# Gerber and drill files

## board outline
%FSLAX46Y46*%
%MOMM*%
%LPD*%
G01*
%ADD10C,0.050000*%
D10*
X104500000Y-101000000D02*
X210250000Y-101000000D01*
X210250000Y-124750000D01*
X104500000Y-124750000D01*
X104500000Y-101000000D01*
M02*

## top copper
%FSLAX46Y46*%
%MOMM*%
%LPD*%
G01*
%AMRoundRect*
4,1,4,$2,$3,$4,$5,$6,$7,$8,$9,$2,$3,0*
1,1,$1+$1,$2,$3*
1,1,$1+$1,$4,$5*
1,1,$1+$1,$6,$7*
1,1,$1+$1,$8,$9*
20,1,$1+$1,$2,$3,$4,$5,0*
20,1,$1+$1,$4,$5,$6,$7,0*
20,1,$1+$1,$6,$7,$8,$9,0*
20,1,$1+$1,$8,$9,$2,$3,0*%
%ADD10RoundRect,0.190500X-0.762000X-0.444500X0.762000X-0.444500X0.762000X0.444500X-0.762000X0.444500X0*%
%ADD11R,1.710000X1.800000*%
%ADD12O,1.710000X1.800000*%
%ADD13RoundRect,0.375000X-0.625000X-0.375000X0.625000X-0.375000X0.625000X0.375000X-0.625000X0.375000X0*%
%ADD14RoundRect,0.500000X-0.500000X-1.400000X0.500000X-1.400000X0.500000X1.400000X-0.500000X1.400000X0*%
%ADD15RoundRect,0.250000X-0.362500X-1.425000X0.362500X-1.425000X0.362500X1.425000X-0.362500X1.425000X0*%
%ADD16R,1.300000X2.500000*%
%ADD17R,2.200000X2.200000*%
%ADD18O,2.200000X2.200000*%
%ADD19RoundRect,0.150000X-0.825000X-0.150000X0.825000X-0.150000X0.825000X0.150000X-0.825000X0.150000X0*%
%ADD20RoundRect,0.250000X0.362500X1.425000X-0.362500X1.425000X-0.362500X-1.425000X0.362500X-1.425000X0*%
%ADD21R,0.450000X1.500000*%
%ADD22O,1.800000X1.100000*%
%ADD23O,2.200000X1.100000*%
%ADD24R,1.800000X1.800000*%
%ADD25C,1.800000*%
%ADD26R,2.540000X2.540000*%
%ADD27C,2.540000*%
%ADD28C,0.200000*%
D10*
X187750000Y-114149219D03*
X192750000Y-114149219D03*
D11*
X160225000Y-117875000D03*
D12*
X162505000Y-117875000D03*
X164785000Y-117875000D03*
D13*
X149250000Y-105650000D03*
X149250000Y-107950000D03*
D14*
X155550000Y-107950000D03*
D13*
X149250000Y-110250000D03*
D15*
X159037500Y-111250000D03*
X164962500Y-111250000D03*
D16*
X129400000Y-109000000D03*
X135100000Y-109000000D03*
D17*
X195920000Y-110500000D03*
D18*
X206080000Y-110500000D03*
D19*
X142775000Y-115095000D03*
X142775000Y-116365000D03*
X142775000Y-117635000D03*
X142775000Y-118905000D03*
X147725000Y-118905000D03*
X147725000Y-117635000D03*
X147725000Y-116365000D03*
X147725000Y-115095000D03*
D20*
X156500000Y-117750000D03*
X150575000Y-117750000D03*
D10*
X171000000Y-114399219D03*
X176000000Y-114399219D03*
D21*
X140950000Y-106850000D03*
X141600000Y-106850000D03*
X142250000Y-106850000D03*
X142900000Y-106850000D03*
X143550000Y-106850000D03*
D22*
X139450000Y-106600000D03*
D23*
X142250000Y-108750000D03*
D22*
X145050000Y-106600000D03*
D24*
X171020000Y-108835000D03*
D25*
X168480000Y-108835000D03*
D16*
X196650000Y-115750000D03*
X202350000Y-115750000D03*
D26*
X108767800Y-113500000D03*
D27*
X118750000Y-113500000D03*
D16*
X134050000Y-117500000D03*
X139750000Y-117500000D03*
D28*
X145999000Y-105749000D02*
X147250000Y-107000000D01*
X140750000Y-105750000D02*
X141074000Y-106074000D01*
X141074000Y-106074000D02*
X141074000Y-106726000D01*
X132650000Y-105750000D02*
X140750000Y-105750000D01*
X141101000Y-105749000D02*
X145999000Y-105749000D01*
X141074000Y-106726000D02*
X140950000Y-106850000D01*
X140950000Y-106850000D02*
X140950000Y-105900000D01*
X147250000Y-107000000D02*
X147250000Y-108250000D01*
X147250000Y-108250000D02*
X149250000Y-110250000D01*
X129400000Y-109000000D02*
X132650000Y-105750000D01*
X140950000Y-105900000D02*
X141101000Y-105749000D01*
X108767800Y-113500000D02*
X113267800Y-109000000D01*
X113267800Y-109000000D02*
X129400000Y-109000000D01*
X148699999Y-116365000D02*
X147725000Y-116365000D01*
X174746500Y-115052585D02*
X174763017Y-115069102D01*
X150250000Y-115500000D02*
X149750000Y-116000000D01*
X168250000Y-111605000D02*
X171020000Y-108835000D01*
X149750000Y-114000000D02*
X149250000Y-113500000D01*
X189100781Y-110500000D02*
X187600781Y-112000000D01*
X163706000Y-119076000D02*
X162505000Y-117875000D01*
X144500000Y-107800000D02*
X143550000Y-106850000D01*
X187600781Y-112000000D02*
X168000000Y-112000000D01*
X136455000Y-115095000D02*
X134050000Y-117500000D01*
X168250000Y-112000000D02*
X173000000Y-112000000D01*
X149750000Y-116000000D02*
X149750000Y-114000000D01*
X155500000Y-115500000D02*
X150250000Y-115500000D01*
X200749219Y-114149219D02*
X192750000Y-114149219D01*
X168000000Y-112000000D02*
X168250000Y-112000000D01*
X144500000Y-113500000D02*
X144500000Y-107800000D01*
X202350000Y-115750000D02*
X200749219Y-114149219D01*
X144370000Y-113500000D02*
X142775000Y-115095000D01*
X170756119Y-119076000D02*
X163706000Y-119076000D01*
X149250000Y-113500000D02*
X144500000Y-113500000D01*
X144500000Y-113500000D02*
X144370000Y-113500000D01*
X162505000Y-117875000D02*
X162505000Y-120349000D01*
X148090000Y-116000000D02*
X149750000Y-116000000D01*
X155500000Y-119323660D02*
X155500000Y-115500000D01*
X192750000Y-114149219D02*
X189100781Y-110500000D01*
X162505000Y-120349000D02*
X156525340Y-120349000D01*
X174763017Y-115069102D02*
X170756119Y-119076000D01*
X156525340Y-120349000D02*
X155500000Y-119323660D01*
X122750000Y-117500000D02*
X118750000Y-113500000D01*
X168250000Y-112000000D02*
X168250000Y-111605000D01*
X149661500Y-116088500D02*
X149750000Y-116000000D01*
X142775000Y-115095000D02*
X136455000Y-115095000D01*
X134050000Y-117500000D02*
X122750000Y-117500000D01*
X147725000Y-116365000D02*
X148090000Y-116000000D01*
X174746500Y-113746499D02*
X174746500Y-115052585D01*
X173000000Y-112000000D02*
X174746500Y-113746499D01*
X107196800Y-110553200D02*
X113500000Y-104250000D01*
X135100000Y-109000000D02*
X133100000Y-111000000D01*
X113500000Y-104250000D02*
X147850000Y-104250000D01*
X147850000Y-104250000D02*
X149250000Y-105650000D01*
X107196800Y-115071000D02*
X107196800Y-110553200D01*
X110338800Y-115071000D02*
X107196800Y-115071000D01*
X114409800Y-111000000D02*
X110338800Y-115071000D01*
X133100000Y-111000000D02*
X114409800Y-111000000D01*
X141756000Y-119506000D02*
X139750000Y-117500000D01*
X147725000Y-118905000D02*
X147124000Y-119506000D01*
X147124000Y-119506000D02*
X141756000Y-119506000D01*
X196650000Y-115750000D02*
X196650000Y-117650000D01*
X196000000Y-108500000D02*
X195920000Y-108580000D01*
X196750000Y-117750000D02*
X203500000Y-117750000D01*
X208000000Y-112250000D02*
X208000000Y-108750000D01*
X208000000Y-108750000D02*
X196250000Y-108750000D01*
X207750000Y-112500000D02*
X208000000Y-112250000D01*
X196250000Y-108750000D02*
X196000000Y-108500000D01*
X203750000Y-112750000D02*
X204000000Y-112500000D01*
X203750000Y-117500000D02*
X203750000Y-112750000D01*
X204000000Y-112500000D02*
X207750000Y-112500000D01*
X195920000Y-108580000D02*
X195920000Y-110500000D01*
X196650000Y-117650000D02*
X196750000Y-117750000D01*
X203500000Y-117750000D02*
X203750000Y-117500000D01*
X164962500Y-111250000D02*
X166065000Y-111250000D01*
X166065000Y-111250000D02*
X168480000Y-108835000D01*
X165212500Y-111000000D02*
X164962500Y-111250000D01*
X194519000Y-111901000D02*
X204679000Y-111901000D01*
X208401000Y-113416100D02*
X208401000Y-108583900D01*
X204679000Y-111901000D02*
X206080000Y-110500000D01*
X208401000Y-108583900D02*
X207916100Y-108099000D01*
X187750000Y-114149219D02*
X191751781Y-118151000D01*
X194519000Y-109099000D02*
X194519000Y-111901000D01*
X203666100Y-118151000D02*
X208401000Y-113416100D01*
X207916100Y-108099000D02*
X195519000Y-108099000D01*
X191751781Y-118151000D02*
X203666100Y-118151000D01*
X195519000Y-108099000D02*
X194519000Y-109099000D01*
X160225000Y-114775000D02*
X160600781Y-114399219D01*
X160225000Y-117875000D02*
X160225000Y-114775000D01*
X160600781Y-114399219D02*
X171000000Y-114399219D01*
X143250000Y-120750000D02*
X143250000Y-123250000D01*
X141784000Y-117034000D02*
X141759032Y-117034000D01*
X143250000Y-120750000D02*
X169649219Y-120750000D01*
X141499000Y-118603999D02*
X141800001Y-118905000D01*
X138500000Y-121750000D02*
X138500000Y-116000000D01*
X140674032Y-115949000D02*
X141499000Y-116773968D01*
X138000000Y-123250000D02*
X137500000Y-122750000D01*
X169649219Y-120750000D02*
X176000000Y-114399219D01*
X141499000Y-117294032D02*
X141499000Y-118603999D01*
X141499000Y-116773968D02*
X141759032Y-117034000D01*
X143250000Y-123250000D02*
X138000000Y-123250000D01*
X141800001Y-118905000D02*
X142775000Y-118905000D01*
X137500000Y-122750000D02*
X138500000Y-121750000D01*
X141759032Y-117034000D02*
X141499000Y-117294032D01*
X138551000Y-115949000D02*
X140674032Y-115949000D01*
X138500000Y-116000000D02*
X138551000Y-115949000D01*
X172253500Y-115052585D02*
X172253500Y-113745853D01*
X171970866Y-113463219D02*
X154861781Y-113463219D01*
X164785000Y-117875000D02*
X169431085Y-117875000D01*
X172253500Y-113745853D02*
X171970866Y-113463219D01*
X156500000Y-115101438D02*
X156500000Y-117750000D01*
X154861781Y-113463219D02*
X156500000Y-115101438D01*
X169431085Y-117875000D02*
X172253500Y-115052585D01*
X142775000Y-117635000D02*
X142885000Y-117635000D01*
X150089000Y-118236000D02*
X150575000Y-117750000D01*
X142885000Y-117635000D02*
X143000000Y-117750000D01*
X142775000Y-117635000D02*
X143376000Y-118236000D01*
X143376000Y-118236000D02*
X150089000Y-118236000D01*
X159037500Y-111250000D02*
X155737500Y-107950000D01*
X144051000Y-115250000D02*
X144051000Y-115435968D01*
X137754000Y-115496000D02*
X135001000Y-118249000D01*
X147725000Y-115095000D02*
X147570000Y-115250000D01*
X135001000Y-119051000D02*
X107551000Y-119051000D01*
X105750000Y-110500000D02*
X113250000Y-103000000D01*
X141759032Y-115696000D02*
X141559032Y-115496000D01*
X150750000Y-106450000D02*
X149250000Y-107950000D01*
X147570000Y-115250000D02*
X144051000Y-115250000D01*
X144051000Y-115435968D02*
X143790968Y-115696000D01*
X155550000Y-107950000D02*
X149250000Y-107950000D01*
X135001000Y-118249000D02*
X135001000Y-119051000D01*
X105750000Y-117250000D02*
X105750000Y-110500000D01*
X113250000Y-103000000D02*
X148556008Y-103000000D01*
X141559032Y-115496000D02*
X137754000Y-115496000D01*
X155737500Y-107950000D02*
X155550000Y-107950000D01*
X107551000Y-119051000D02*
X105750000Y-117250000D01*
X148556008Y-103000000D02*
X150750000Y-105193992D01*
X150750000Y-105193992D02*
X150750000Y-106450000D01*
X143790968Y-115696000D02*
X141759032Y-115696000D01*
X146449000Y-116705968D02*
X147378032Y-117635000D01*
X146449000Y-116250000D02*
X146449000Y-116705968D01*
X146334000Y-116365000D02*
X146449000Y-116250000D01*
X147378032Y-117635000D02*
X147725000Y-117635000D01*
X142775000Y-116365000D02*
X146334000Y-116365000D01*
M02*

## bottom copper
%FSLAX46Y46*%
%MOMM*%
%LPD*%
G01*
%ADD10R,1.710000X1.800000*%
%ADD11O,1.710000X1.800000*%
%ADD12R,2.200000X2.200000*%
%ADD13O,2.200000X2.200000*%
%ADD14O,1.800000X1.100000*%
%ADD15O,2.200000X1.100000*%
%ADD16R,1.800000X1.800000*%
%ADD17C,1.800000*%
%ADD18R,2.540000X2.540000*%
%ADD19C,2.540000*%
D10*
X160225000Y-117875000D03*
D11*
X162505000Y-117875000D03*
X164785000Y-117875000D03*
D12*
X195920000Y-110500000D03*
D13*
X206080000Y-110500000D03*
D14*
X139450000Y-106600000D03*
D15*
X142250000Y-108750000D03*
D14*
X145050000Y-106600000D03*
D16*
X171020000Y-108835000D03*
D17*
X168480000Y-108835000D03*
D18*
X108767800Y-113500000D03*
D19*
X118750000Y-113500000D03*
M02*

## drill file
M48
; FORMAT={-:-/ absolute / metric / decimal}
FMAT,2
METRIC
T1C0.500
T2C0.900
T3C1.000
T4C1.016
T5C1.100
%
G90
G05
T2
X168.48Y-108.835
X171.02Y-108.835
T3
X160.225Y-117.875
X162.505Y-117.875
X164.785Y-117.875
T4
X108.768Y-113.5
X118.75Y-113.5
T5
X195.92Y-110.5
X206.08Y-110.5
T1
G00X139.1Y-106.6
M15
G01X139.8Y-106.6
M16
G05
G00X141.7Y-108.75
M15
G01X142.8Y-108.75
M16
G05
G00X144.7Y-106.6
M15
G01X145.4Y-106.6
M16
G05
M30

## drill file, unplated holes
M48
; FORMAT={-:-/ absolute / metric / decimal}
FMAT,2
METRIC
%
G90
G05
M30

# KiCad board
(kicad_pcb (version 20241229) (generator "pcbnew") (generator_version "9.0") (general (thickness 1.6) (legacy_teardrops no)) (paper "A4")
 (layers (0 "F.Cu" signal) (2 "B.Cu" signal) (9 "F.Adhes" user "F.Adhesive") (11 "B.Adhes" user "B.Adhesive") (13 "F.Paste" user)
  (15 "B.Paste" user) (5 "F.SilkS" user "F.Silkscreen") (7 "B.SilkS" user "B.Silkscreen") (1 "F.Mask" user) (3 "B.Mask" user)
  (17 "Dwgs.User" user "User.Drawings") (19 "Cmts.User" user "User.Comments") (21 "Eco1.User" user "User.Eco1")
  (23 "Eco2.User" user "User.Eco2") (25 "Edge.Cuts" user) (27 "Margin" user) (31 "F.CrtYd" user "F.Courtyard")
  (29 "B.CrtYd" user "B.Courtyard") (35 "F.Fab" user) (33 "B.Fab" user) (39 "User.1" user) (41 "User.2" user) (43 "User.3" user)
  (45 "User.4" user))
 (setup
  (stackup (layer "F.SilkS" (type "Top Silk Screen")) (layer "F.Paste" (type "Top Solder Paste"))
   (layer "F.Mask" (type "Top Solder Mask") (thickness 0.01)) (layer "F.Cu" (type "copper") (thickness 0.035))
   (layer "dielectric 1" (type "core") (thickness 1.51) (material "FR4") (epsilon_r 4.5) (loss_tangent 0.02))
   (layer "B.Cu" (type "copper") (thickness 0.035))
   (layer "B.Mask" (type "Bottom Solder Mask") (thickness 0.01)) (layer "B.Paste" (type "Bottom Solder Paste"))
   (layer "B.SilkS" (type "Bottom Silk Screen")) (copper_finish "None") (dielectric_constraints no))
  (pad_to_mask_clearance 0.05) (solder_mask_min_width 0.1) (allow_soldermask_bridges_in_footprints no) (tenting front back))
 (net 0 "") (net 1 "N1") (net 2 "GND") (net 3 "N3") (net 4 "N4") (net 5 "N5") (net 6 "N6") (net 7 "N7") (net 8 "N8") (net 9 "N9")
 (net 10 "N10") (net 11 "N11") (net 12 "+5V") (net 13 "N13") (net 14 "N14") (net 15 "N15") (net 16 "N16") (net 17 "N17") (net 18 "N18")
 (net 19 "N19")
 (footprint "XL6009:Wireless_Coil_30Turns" (layer "F.Cu") (at 190.25 109.149219)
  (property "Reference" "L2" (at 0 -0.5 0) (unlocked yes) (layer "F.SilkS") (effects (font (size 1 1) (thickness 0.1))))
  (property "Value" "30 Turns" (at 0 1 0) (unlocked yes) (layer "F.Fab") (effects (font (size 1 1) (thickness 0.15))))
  (pad "1" smd roundrect (at -2.5 5) (size 1.905 1.27) (layers "F.Cu" "F.Mask" "F.Paste") (roundrect_rratio 0.15) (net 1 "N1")
   (thermal_bridge_angle 45))
  (pad "2" smd roundrect (at 2.5 5) (size 1.905 1.27) (layers "F.Cu" "F.Mask" "F.Paste") (roundrect_rratio 0.15) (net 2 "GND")
   (thermal_bridge_angle 45)))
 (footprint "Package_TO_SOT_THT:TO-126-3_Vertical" (layer "F.Cu") (at 160.225 117.875)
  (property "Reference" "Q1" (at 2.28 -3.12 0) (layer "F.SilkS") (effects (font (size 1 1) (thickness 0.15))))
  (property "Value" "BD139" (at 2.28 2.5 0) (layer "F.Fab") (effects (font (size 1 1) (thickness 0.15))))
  (pad "1" thru_hole rect (at 0 0) (size 1.71 1.8) (drill 1) (layers "*.Cu" "*.Mask") (remove_unused_layers no) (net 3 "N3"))
  (pad "2" thru_hole oval (at 2.28 0) (size 1.71 1.8) (drill 1) (layers "*.Cu" "*.Mask") (remove_unused_layers no) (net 2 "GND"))
  (pad "3" thru_hole oval (at 4.56 0) (size 1.71 1.8) (drill 1) (layers "*.Cu" "*.Mask") (remove_unused_layers no) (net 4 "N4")))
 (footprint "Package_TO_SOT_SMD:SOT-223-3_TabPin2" (layer "F.Cu") (at 152.4 107.95)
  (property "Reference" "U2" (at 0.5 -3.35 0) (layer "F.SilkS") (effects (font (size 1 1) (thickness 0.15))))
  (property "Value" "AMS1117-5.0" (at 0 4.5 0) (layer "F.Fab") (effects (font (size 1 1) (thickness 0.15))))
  (pad "1" smd roundrect (at -3.15 -2.3) (size 2 1.5) (layers "F.Cu" "F.Mask" "F.Paste") (roundrect_rratio 0.25) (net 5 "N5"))
  (pad "2" smd roundrect (at -3.15 0) (size 2 1.5) (layers "F.Cu" "F.Mask" "F.Paste") (roundrect_rratio 0.25) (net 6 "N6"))
  (pad "2" smd roundrect (at 3.15 0) (size 2 3.8) (layers "F.Cu" "F.Mask" "F.Paste") (roundrect_rratio 0.25) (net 6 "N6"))
  (pad "3" smd roundrect (at -3.15 2.3) (size 2 1.5) (layers "F.Cu" "F.Mask" "F.Paste") (roundrect_rratio 0.25) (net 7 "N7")))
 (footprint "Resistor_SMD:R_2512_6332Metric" (layer "F.Cu") (at 162 111.25)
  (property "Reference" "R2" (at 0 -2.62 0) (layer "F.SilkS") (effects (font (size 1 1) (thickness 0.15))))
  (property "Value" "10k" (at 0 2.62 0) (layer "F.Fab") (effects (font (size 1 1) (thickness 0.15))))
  (pad "1" smd roundrect (at -2.9625 0) (size 1.225 3.35) (layers "F.Cu" "F.Mask" "F.Paste") (roundrect_rratio 0.204082) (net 6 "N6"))
  (pad "2" smd roundrect (at 2.9625 0) (size 1.225 3.35) (layers "F.Cu" "F.Mask" "F.Paste") (roundrect_rratio 0.204082) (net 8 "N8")))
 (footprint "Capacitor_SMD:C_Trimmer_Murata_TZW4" (layer "F.Cu") (at 132.25 109)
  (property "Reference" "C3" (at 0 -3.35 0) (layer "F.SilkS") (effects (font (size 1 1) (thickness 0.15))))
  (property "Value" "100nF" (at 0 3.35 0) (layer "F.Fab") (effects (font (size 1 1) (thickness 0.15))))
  (pad "1" smd rect (at -2.85 0) (size 1.3 2.5) (layers "F.Cu" "F.Mask" "F.Paste") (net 7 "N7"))
  (pad "2" smd rect (at 2.85 0) (size 1.3 2.5) (layers "F.Cu" "F.Mask" "F.Paste") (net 5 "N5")))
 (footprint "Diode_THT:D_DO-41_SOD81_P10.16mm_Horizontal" (layer "F.Cu") (at 195.92 110.5)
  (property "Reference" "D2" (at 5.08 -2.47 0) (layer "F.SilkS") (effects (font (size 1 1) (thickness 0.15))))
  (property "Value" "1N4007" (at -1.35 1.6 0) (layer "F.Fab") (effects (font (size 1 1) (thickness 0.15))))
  (pad "1" thru_hole rect (at 0 0) (size 2.2 2.2) (drill 1.1) (layers "*.Cu" "*.Mask") (remove_unused_layers no) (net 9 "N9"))
  (pad "2" thru_hole oval (at 10.16 0) (size 2.2 2.2) (drill 1.1) (layers "*.Cu" "*.Mask") (remove_unused_layers no) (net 1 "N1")))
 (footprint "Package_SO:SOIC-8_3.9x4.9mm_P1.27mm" (layer "F.Cu") (at 145.25 117)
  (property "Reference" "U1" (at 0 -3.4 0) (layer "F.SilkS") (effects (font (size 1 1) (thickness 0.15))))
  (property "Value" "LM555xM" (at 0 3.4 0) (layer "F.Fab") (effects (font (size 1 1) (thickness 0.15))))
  (pad "1" smd roundrect (at -2.475 -1.905) (size 1.95 0.6) (layers "F.Cu" "F.Mask" "F.Paste") (roundrect_rratio 0.25) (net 2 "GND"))
  (pad "2" smd roundrect (at -2.475 -0.635) (size 1.95 0.6) (layers "F.Cu" "F.Mask" "F.Paste") (roundrect_rratio 0.25) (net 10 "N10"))
  (pad "3" smd roundrect (at -2.475 0.635) (size 1.95 0.6) (layers "F.Cu" "F.Mask" "F.Paste") (roundrect_rratio 0.25) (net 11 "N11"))
  (pad "4" smd roundrect (at -2.475 1.905) (size 1.95 0.6) (layers "F.Cu" "F.Mask" "F.Paste") (roundrect_rratio 0.25) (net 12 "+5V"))
  (pad "5" smd roundrect (at 2.475 1.905) (size 1.95 0.6) (layers "F.Cu" "F.Mask" "F.Paste") (roundrect_rratio 0.25) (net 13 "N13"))
  (pad "6" smd roundrect (at 2.475 0.635) (size 1.95 0.6) (layers "F.Cu" "F.Mask" "F.Paste") (roundrect_rratio 0.25) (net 10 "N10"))
  (pad "7" smd roundrect (at 2.475 -0.635) (size 1.95 0.6) (layers "F.Cu" "F.Mask" "F.Paste") (roundrect_rratio 0.25) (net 2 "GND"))
  (pad "8" smd roundrect (at 2.475 -1.905) (size 1.95 0.6) (layers "F.Cu" "F.Mask" "F.Paste") (roundrect_rratio 0.25) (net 6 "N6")))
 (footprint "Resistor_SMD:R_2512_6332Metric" (layer "F.Cu") (at 153.5375 117.75 180)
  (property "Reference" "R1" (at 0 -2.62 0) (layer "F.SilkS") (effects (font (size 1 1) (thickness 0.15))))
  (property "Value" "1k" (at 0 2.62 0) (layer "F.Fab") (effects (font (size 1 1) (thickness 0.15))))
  (pad "1" smd roundrect (at -2.9625 0 180) (size 1.225 3.35) (layers "F.Cu" "F.Mask" "F.Paste") (roundrect_rratio 0.204082) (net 4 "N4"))
  (pad "2" smd roundrect (at 2.9625 0 180) (size 1.225 3.35) (layers "F.Cu" "F.Mask" "F.Paste") (roundrect_rratio 0.204082) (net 11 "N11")))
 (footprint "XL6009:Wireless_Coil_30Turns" (layer "F.Cu") (at 173.5 109.399219)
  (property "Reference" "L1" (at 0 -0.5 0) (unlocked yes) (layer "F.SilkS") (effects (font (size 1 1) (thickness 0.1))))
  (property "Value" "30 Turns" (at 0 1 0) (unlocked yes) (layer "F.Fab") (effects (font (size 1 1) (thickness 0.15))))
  (pad "1" smd roundrect (at -2.5 5) (size 1.905 1.27) (layers "F.Cu" "F.Mask" "F.Paste") (roundrect_rratio 0.15) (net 3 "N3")
   (thermal_bridge_angle 45))
  (pad "2" smd roundrect (at 2.5 5) (size 1.905 1.27) (layers "F.Cu" "F.Mask" "F.Paste") (roundrect_rratio 0.15) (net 12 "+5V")
   (thermal_bridge_angle 45)))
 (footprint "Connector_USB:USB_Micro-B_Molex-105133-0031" (layer "F.Cu") (at 142.25 107.675)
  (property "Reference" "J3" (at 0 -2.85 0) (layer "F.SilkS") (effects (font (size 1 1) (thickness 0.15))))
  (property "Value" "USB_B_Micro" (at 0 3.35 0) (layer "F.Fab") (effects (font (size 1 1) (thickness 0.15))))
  (pad "1" smd rect (at -1.3 -0.825) (size 0.45 1.5) (layers "F.Cu" "F.Mask" "F.Paste") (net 7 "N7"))
  (pad "2" smd rect (at -0.65 -0.825) (size 0.45 1.5) (layers "F.Cu" "F.Mask" "F.Paste") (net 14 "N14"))
  (pad "3" smd rect (at 0 -0.825) (size 0.45 1.5) (layers "F.Cu" "F.Mask" "F.Paste") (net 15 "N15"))
  (pad "4" smd rect (at 0.65 -0.825) (size 0.45 1.5) (layers "F.Cu" "F.Mask" "F.Paste") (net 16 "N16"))
  (pad "5" smd rect (at 1.3 -0.825) (size 0.45 1.5) (layers "F.Cu" "F.Mask" "F.Paste") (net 2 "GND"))
  (pad "6" thru_hole oval (at -2.8 -1.075) (size 1.8 1.1) (drill oval 1.2 0.5) (layers "*.Cu" "*.Mask") (remove_unused_layers no)
   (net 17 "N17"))
  (pad "6" thru_hole oval (at 0 1.075) (size 2.2 1.1) (drill oval 1.6 0.5) (layers "*.Cu" "*.Mask") (remove_unused_layers no) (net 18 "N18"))
  (pad "6" thru_hole oval (at 2.8 -1.075) (size 1.8 1.1) (drill oval 1.2 0.5) (layers "*.Cu" "*.Mask") (remove_unused_layers no)
   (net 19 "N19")))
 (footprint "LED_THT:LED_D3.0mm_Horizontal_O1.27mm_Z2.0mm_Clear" (layer "F.Cu") (at 171.02 108.835 180)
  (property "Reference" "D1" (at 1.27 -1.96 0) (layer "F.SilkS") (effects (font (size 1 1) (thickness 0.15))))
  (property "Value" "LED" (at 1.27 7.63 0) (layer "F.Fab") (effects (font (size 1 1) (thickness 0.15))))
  (pad "1" thru_hole rect (at 0 0 180) (size 1.8 1.8) (drill 0.9) (layers "*.Cu" "*.Mask") (remove_unused_layers no) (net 2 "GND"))
  (pad "2" thru_hole circle (at 2.54 0 180) (size 1.8 1.8) (drill 0.9) (layers "*.Cu" "*.Mask") (remove_unused_layers no) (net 8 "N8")))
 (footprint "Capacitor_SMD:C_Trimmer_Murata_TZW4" (layer "F.Cu") (at 199.5 115.75)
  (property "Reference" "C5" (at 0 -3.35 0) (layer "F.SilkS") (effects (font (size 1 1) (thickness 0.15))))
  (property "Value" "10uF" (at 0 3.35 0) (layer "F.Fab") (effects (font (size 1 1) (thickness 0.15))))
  (pad "1" smd rect (at -2.85 0) (size 1.3 2.5) (layers "F.Cu" "F.Mask" "F.Paste") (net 9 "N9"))
  (pad "2" smd rect (at 2.85 0) (size 1.3 2.5) (layers "F.Cu" "F.Mask" "F.Paste") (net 2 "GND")))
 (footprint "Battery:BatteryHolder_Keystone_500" (layer "F.Cu") (at 108.7678 113.5)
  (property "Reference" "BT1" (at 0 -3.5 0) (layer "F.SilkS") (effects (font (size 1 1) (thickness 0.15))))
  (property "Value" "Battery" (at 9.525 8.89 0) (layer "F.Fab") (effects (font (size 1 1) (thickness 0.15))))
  (pad "1" thru_hole rect (at 0 0) (size 2.54 2.54) (drill 1.016) (layers "*.Cu" "*.Mask") (remove_unused_layers no) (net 7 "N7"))
  (pad "2" thru_hole circle (at 9.9822 0) (size 2.54 2.54) (drill 1.016) (layers "*.Cu" "*.Mask") (remove_unused_layers no) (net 2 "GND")))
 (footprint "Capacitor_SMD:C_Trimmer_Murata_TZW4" (layer "F.Cu") (at 136.9 117.5)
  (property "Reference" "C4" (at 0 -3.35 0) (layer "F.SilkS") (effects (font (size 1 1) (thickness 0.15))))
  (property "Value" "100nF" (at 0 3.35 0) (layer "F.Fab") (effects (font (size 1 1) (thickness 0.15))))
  (pad "1" smd rect (at -2.85 0) (size 1.3 2.5) (layers "F.Cu" "F.Mask" "F.Paste") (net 2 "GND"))
  (pad "2" smd rect (at 2.85 0) (size 1.3 2.5) (layers "F.Cu" "F.Mask" "F.Paste") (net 13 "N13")))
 (gr_rect (start 104.5 101) (end 210.25 124.75) (stroke (width 0.05) (type default)) (fill no) (layer "Edge.Cuts"))
 (segment (start 145.999 105.749) (end 147.25 107) (width 0.2) (layer "F.Cu") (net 7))
 (segment (start 140.75 105.75) (end 141.074 106.074) (width 0.2) (layer "F.Cu") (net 7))
 (segment (start 141.074 106.074) (end 141.074 106.726) (width 0.2) (layer "F.Cu") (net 7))
 (segment (start 132.65 105.75) (end 140.75 105.75) (width 0.2) (layer "F.Cu") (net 7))
 (segment (start 141.101 105.749) (end 145.999 105.749) (width 0.2) (layer "F.Cu") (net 7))
 (segment (start 141.074 106.726) (end 140.95 106.85) (width 0.2) (layer "F.Cu") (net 7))
 (segment (start 140.95 106.85) (end 140.95 105.9) (width 0.2) (layer "F.Cu") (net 7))
 (segment (start 147.25 107) (end 147.25 108.25) (width 0.2) (layer "F.Cu") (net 7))
 (segment (start 147.25 108.25) (end 149.25 110.25) (width 0.2) (layer "F.Cu") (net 7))
 (segment (start 129.4 109) (end 132.65 105.75) (width 0.2) (layer "F.Cu") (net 7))
 (segment (start 140.95 105.9) (end 141.101 105.749) (width 0.2) (layer "F.Cu") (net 7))
 (segment (start 108.7678 113.5) (end 113.2678 109) (width 0.2) (layer "F.Cu") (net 7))
 (segment (start 113.2678 109) (end 129.4 109) (width 0.2) (layer "F.Cu") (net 7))
 (segment (start 148.699999 116.365) (end 147.725 116.365) (width 0.2) (layer "F.Cu") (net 2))
 (segment (start 174.7465 115.052585) (end 174.763017 115.069102) (width 0.2) (layer "F.Cu") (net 2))
 (segment (start 150.25 115.5) (end 149.75 116) (width 0.2) (layer "F.Cu") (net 2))
 (segment (start 168.25 111.605) (end 171.02 108.835) (width 0.2) (layer "F.Cu") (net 2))
 (segment (start 149.75 114) (end 149.25 113.5) (width 0.2) (layer "F.Cu") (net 2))
 (segment (start 189.100781 110.5) (end 187.600781 112) (width 0.2) (layer "F.Cu") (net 2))
 (segment (start 163.706 119.076) (end 162.505 117.875) (width 0.2) (layer "F.Cu") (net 2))
 (segment (start 144.5 107.8) (end 143.55 106.85) (width 0.2) (layer "F.Cu") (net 2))
 (segment (start 187.600781 112) (end 168 112) (width 0.2) (layer "F.Cu") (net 2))
 (segment (start 136.455 115.095) (end 134.05 117.5) (width 0.2) (layer "F.Cu") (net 2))
 (segment (start 168.25 112) (end 173 112) (width 0.2) (layer "F.Cu") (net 2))
 (segment (start 149.75 116) (end 149.75 114) (width 0.2) (layer "F.Cu") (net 2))
 (segment (start 155.5 115.5) (end 150.25 115.5) (width 0.2) (layer "F.Cu") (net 2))
 (segment (start 200.749219 114.149219) (end 192.75 114.149219) (width 0.2) (layer "F.Cu") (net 2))
 (segment (start 168 112) (end 168.25 112) (width 0.2) (layer "F.Cu") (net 2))
 (segment (start 144.5 113.5) (end 144.5 107.8) (width 0.2) (layer "F.Cu") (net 2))
 (segment (start 202.35 115.75) (end 200.749219 114.149219) (width 0.2) (layer "F.Cu") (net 2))
 (segment (start 144.37 113.5) (end 142.775 115.095) (width 0.2) (layer "F.Cu") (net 2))
 (segment (start 170.756119 119.076) (end 163.706 119.076) (width 0.2) (layer "F.Cu") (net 2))
 (segment (start 149.25 113.5) (end 144.5 113.5) (width 0.2) (layer "F.Cu") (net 2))
 (segment (start 144.5 113.5) (end 144.37 113.5) (width 0.2) (layer "F.Cu") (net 2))
 (segment (start 162.505 117.875) (end 162.505 120.349) (width 0.2) (layer "F.Cu") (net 2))
 (segment (start 148.09 116) (end 149.75 116) (width 0.2) (layer "F.Cu") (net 2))
 (segment (start 155.5 119.32366) (end 155.5 115.5) (width 0.2) (layer "F.Cu") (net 2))
 (segment (start 192.75 114.149219) (end 189.100781 110.5) (width 0.2) (layer "F.Cu") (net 2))
 (segment (start 162.505 120.349) (end 156.52534 120.349) (width 0.2) (layer "F.Cu") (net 2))
 (segment (start 174.763017 115.069102) (end 170.756119 119.076) (width 0.2) (layer "F.Cu") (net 2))
 (segment (start 156.52534 120.349) (end 155.5 119.32366) (width 0.2) (layer "F.Cu") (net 2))
 (segment (start 122.75 117.5) (end 118.75 113.5) (width 0.2) (layer "F.Cu") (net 2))
 (segment (start 168.25 112) (end 168.25 111.605) (width 0.2) (layer "F.Cu") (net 2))
 (segment (start 149.6615 116.0885) (end 149.75 116) (width 0.2) (layer "F.Cu") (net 2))
 (segment (start 142.775 115.095) (end 136.455 115.095) (width 0.2) (layer "F.Cu") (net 2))
 (segment (start 134.05 117.5) (end 122.75 117.5) (width 0.2) (layer "F.Cu") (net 2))
 (segment (start 147.725 116.365) (end 148.09 116) (width 0.2) (layer "F.Cu") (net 2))
 (segment (start 174.7465 113.746499) (end 174.7465 115.052585) (width 0.2) (layer "F.Cu") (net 2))
 (segment (start 173 112) (end 174.7465 113.746499) (width 0.2) (layer "F.Cu") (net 2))
 (segment (start 107.1968 110.5532) (end 113.5 104.25) (width 0.2) (layer "F.Cu") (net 5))
 (segment (start 135.1 109) (end 133.1 111) (width 0.2) (layer "F.Cu") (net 5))
 (segment (start 113.5 104.25) (end 147.85 104.25) (width 0.2) (layer "F.Cu") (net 5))
 (segment (start 147.85 104.25) (end 149.25 105.65) (width 0.2) (layer "F.Cu") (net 5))
 (segment (start 107.1968 115.071) (end 107.1968 110.5532) (width 0.2) (layer "F.Cu") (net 5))
 (segment (start 110.3388 115.071) (end 107.1968 115.071) (width 0.2) (layer "F.Cu") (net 5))
 (segment (start 114.4098 111) (end 110.3388 115.071) (width 0.2) (layer "F.Cu") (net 5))
 (segment (start 133.1 111) (end 114.4098 111) (width 0.2) (layer "F.Cu") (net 5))
 (segment (start 141.756 119.506) (end 139.75 117.5) (width 0.2) (layer "F.Cu") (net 13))
 (segment (start 147.725 118.905) (end 147.124 119.506) (width 0.2) (layer "F.Cu") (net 13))
 (segment (start 147.124 119.506) (end 141.756 119.506) (width 0.2) (layer "F.Cu") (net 13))
 (segment (start 196.65 115.75) (end 196.65 117.65) (width 0.2) (layer "F.Cu") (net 9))
 (segment (start 196 108.5) (end 195.92 108.58) (width 0.2) (layer "F.Cu") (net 9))
 (segment (start 196.75 117.75) (end 203.5 117.75) (width 0.2) (layer "F.Cu") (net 9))
 (segment (start 208 112.25) (end 208 108.75) (width 0.2) (layer "F.Cu") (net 9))
 (segment (start 208 108.75) (end 196.25 108.75) (width 0.2) (layer "F.Cu") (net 9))
 (segment (start 207.75 112.5) (end 208 112.25) (width 0.2) (layer "F.Cu") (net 9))
 (segment (start 196.25 108.75) (end 196 108.5) (width 0.2) (layer "F.Cu") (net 9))
 (segment (start 203.75 112.75) (end 204 112.5) (width 0.2) (layer "F.Cu") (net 9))
 (segment (start 203.75 117.5) (end 203.75 112.75) (width 0.2) (layer "F.Cu") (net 9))
 (segment (start 204 112.5) (end 207.75 112.5) (width 0.2) (layer "F.Cu") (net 9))
 (segment (start 195.92 108.58) (end 195.92 110.5) (width 0.2) (layer "F.Cu") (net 9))
 (segment (start 196.65 117.65) (end 196.75 117.75) (width 0.2) (layer "F.Cu") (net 9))
 (segment (start 203.5 117.75) (end 203.75 117.5) (width 0.2) (layer "F.Cu") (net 9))
 (segment (start 164.9625 111.25) (end 166.065 111.25) (width 0.2) (layer "F.Cu") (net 8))
 (segment (start 166.065 111.25) (end 168.48 108.835) (width 0.2) (layer "F.Cu") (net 8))
 (segment (start 165.2125 111) (end 164.9625 111.25) (width 0.2) (layer "F.Cu") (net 8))
 (segment (start 194.519 111.901) (end 204.679 111.901) (width 0.2) (layer "F.Cu") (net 1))
 (segment (start 208.401 113.4161) (end 208.401 108.5839) (width 0.2) (layer "F.Cu") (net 1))
 (segment (start 204.679 111.901) (end 206.08 110.5) (width 0.2) (layer "F.Cu") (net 1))
 (segment (start 208.401 108.5839) (end 207.9161 108.099) (width 0.2) (layer "F.Cu") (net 1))
 (segment (start 187.75 114.149219) (end 191.751781 118.151) (width 0.2) (layer "F.Cu") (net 1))
 (segment (start 194.519 109.099) (end 194.519 111.901) (width 0.2) (layer "F.Cu") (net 1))
 (segment (start 203.6661 118.151) (end 208.401 113.4161) (width 0.2) (layer "F.Cu") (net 1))
 (segment (start 207.9161 108.099) (end 195.519 108.099) (width 0.2) (layer "F.Cu") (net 1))
 (segment (start 191.751781 118.151) (end 203.6661 118.151) (width 0.2) (layer "F.Cu") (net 1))
 (segment (start 195.519 108.099) (end 194.519 109.099) (width 0.2) (layer "F.Cu") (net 1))
 (segment (start 160.225 114.775) (end 160.600781 114.399219) (width 0.2) (layer "F.Cu") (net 3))
 (segment (start 160.225 117.875) (end 160.225 114.775) (width 0.2) (layer "F.Cu") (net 3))
 (segment (start 160.600781 114.399219) (end 171 114.399219) (width 0.2) (layer "F.Cu") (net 3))
 (segment (start 143.25 120.75) (end 143.25 123.25) (width 0.2) (layer "F.Cu") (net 12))
 (segment (start 141.784 117.034) (end 141.759032 117.034) (width 0.2) (layer "F.Cu") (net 12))
 (segment (start 143.25 120.75) (end 169.649219 120.75) (width 0.2) (layer "F.Cu") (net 12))
 (segment (start 141.499 118.603999) (end 141.800001 118.905) (width 0.2) (layer "F.Cu") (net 12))
 (segment (start 138.5 121.75) (end 138.5 116) (width 0.2) (layer "F.Cu") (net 12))
 (segment (start 140.674032 115.949) (end 141.499 116.773968) (width 0.2) (layer "F.Cu") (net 12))
 (segment (start 138 123.25) (end 137.5 122.75) (width 0.2) (layer "F.Cu") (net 12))
 (segment (start 169.649219 120.75) (end 176 114.399219) (width 0.2) (layer "F.Cu") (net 12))
 (segment (start 141.499 117.294032) (end 141.499 118.603999) (width 0.2) (layer "F.Cu") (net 12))
 (segment (start 141.499 116.773968) (end 141.759032 117.034) (width 0.2) (layer "F.Cu") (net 12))
 (segment (start 143.25 123.25) (end 138 123.25) (width 0.2) (layer "F.Cu") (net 12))
 (segment (start 141.800001 118.905) (end 142.775 118.905) (width 0.2) (layer "F.Cu") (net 12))
 (segment (start 137.5 122.75) (end 138.5 121.75) (width 0.2) (layer "F.Cu") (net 12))
 (segment (start 141.759032 117.034) (end 141.499 117.294032) (width 0.2) (layer "F.Cu") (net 12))
 (segment (start 138.551 115.949) (end 140.674032 115.949) (width 0.2) (layer "F.Cu") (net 12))
 (segment (start 138.5 116) (end 138.551 115.949) (width 0.2) (layer "F.Cu") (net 12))
 (segment (start 172.2535 115.052585) (end 172.2535 113.745853) (width 0.2) (layer "F.Cu") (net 4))
 (segment (start 171.970866 113.463219) (end 154.861781 113.463219) (width 0.2) (layer "F.Cu") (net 4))
 (segment (start 164.785 117.875) (end 169.431085 117.875) (width 0.2) (layer "F.Cu") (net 4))
 (segment (start 172.2535 113.745853) (end 171.970866 113.463219) (width 0.2) (layer "F.Cu") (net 4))
 (segment (start 156.5 115.101438) (end 156.5 117.75) (width 0.2) (layer "F.Cu") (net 4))
 (segment (start 154.861781 113.463219) (end 156.5 115.101438) (width 0.2) (layer "F.Cu") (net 4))
 (segment (start 169.431085 117.875) (end 172.2535 115.052585) (width 0.2) (layer "F.Cu") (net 4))
 (segment (start 142.775 117.635) (end 142.885 117.635) (width 0.2) (layer "F.Cu") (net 11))
 (segment (start 150.089 118.236) (end 150.575 117.75) (width 0.2) (layer "F.Cu") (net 11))
 (segment (start 142.885 117.635) (end 143 117.75) (width 0.2) (layer "F.Cu") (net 11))
 (segment (start 142.775 117.635) (end 143.376 118.236) (width 0.2) (layer "F.Cu") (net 11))
 (segment (start 143.376 118.236) (end 150.089 118.236) (width 0.2) (layer "F.Cu") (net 11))
 (segment (start 159.0375 111.25) (end 155.7375 107.95) (width 0.2) (layer "F.Cu") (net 6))
 (segment (start 144.051 115.25) (end 144.051 115.435968) (width 0.2) (layer "F.Cu") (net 6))
 (segment (start 137.754 115.496) (end 135.001 118.249) (width 0.2) (layer "F.Cu") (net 6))
 (segment (start 147.725 115.095) (end 147.57 115.25) (width 0.2) (layer "F.Cu") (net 6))
 (segment (start 135.001 119.051) (end 107.551 119.051) (width 0.2) (layer "F.Cu") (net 6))
 (segment (start 105.75 110.5) (end 113.25 103) (width 0.2) (layer "F.Cu") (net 6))
 (segment (start 141.759032 115.696) (end 141.559032 115.496) (width 0.2) (layer "F.Cu") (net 6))
 (segment (start 150.75 106.45) (end 149.25 107.95) (width 0.2) (layer "F.Cu") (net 6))
 (segment (start 147.57 115.25) (end 144.051 115.25) (width 0.2) (layer "F.Cu") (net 6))
 (segment (start 144.051 115.435968) (end 143.790968 115.696) (width 0.2) (layer "F.Cu") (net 6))
 (segment (start 155.55 107.95) (end 149.25 107.95) (width 0.2) (layer "F.Cu") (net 6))
 (segment (start 135.001 118.249) (end 135.001 119.051) (width 0.2) (layer "F.Cu") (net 6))
 (segment (start 105.75 117.25) (end 105.75 110.5) (width 0.2) (layer "F.Cu") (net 6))
 (segment (start 113.25 103) (end 148.556008 103) (width 0.2) (layer "F.Cu") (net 6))
 (segment (start 141.559032 115.496) (end 137.754 115.496) (width 0.2) (layer "F.Cu") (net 6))
 (segment (start 155.7375 107.95) (end 155.55 107.95) (width 0.2) (layer "F.Cu") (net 6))
 (segment (start 107.551 119.051) (end 105.75 117.25) (width 0.2) (layer "F.Cu") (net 6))
 (segment (start 148.556008 103) (end 150.75 105.193992) (width 0.2) (layer "F.Cu") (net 6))
 (segment (start 150.75 105.193992) (end 150.75 106.45) (width 0.2) (layer "F.Cu") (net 6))
 (segment (start 143.790968 115.696) (end 141.759032 115.696) (width 0.2) (layer "F.Cu") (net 6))
 (segment (start 146.449 116.705968) (end 147.378032 117.635) (width 0.2) (layer "F.Cu") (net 10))
 (segment (start 146.449 116.25) (end 146.449 116.705968) (width 0.2) (layer "F.Cu") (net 10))
 (segment (start 146.334 116.365) (end 146.449 116.25) (width 0.2) (layer "F.Cu") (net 10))
 (segment (start 147.378032 117.635) (end 147.725 117.635) (width 0.2) (layer "F.Cu") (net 10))
 (segment (start 142.775 116.365) (end 146.334 116.365) (width 0.2) (layer "F.Cu") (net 10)))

